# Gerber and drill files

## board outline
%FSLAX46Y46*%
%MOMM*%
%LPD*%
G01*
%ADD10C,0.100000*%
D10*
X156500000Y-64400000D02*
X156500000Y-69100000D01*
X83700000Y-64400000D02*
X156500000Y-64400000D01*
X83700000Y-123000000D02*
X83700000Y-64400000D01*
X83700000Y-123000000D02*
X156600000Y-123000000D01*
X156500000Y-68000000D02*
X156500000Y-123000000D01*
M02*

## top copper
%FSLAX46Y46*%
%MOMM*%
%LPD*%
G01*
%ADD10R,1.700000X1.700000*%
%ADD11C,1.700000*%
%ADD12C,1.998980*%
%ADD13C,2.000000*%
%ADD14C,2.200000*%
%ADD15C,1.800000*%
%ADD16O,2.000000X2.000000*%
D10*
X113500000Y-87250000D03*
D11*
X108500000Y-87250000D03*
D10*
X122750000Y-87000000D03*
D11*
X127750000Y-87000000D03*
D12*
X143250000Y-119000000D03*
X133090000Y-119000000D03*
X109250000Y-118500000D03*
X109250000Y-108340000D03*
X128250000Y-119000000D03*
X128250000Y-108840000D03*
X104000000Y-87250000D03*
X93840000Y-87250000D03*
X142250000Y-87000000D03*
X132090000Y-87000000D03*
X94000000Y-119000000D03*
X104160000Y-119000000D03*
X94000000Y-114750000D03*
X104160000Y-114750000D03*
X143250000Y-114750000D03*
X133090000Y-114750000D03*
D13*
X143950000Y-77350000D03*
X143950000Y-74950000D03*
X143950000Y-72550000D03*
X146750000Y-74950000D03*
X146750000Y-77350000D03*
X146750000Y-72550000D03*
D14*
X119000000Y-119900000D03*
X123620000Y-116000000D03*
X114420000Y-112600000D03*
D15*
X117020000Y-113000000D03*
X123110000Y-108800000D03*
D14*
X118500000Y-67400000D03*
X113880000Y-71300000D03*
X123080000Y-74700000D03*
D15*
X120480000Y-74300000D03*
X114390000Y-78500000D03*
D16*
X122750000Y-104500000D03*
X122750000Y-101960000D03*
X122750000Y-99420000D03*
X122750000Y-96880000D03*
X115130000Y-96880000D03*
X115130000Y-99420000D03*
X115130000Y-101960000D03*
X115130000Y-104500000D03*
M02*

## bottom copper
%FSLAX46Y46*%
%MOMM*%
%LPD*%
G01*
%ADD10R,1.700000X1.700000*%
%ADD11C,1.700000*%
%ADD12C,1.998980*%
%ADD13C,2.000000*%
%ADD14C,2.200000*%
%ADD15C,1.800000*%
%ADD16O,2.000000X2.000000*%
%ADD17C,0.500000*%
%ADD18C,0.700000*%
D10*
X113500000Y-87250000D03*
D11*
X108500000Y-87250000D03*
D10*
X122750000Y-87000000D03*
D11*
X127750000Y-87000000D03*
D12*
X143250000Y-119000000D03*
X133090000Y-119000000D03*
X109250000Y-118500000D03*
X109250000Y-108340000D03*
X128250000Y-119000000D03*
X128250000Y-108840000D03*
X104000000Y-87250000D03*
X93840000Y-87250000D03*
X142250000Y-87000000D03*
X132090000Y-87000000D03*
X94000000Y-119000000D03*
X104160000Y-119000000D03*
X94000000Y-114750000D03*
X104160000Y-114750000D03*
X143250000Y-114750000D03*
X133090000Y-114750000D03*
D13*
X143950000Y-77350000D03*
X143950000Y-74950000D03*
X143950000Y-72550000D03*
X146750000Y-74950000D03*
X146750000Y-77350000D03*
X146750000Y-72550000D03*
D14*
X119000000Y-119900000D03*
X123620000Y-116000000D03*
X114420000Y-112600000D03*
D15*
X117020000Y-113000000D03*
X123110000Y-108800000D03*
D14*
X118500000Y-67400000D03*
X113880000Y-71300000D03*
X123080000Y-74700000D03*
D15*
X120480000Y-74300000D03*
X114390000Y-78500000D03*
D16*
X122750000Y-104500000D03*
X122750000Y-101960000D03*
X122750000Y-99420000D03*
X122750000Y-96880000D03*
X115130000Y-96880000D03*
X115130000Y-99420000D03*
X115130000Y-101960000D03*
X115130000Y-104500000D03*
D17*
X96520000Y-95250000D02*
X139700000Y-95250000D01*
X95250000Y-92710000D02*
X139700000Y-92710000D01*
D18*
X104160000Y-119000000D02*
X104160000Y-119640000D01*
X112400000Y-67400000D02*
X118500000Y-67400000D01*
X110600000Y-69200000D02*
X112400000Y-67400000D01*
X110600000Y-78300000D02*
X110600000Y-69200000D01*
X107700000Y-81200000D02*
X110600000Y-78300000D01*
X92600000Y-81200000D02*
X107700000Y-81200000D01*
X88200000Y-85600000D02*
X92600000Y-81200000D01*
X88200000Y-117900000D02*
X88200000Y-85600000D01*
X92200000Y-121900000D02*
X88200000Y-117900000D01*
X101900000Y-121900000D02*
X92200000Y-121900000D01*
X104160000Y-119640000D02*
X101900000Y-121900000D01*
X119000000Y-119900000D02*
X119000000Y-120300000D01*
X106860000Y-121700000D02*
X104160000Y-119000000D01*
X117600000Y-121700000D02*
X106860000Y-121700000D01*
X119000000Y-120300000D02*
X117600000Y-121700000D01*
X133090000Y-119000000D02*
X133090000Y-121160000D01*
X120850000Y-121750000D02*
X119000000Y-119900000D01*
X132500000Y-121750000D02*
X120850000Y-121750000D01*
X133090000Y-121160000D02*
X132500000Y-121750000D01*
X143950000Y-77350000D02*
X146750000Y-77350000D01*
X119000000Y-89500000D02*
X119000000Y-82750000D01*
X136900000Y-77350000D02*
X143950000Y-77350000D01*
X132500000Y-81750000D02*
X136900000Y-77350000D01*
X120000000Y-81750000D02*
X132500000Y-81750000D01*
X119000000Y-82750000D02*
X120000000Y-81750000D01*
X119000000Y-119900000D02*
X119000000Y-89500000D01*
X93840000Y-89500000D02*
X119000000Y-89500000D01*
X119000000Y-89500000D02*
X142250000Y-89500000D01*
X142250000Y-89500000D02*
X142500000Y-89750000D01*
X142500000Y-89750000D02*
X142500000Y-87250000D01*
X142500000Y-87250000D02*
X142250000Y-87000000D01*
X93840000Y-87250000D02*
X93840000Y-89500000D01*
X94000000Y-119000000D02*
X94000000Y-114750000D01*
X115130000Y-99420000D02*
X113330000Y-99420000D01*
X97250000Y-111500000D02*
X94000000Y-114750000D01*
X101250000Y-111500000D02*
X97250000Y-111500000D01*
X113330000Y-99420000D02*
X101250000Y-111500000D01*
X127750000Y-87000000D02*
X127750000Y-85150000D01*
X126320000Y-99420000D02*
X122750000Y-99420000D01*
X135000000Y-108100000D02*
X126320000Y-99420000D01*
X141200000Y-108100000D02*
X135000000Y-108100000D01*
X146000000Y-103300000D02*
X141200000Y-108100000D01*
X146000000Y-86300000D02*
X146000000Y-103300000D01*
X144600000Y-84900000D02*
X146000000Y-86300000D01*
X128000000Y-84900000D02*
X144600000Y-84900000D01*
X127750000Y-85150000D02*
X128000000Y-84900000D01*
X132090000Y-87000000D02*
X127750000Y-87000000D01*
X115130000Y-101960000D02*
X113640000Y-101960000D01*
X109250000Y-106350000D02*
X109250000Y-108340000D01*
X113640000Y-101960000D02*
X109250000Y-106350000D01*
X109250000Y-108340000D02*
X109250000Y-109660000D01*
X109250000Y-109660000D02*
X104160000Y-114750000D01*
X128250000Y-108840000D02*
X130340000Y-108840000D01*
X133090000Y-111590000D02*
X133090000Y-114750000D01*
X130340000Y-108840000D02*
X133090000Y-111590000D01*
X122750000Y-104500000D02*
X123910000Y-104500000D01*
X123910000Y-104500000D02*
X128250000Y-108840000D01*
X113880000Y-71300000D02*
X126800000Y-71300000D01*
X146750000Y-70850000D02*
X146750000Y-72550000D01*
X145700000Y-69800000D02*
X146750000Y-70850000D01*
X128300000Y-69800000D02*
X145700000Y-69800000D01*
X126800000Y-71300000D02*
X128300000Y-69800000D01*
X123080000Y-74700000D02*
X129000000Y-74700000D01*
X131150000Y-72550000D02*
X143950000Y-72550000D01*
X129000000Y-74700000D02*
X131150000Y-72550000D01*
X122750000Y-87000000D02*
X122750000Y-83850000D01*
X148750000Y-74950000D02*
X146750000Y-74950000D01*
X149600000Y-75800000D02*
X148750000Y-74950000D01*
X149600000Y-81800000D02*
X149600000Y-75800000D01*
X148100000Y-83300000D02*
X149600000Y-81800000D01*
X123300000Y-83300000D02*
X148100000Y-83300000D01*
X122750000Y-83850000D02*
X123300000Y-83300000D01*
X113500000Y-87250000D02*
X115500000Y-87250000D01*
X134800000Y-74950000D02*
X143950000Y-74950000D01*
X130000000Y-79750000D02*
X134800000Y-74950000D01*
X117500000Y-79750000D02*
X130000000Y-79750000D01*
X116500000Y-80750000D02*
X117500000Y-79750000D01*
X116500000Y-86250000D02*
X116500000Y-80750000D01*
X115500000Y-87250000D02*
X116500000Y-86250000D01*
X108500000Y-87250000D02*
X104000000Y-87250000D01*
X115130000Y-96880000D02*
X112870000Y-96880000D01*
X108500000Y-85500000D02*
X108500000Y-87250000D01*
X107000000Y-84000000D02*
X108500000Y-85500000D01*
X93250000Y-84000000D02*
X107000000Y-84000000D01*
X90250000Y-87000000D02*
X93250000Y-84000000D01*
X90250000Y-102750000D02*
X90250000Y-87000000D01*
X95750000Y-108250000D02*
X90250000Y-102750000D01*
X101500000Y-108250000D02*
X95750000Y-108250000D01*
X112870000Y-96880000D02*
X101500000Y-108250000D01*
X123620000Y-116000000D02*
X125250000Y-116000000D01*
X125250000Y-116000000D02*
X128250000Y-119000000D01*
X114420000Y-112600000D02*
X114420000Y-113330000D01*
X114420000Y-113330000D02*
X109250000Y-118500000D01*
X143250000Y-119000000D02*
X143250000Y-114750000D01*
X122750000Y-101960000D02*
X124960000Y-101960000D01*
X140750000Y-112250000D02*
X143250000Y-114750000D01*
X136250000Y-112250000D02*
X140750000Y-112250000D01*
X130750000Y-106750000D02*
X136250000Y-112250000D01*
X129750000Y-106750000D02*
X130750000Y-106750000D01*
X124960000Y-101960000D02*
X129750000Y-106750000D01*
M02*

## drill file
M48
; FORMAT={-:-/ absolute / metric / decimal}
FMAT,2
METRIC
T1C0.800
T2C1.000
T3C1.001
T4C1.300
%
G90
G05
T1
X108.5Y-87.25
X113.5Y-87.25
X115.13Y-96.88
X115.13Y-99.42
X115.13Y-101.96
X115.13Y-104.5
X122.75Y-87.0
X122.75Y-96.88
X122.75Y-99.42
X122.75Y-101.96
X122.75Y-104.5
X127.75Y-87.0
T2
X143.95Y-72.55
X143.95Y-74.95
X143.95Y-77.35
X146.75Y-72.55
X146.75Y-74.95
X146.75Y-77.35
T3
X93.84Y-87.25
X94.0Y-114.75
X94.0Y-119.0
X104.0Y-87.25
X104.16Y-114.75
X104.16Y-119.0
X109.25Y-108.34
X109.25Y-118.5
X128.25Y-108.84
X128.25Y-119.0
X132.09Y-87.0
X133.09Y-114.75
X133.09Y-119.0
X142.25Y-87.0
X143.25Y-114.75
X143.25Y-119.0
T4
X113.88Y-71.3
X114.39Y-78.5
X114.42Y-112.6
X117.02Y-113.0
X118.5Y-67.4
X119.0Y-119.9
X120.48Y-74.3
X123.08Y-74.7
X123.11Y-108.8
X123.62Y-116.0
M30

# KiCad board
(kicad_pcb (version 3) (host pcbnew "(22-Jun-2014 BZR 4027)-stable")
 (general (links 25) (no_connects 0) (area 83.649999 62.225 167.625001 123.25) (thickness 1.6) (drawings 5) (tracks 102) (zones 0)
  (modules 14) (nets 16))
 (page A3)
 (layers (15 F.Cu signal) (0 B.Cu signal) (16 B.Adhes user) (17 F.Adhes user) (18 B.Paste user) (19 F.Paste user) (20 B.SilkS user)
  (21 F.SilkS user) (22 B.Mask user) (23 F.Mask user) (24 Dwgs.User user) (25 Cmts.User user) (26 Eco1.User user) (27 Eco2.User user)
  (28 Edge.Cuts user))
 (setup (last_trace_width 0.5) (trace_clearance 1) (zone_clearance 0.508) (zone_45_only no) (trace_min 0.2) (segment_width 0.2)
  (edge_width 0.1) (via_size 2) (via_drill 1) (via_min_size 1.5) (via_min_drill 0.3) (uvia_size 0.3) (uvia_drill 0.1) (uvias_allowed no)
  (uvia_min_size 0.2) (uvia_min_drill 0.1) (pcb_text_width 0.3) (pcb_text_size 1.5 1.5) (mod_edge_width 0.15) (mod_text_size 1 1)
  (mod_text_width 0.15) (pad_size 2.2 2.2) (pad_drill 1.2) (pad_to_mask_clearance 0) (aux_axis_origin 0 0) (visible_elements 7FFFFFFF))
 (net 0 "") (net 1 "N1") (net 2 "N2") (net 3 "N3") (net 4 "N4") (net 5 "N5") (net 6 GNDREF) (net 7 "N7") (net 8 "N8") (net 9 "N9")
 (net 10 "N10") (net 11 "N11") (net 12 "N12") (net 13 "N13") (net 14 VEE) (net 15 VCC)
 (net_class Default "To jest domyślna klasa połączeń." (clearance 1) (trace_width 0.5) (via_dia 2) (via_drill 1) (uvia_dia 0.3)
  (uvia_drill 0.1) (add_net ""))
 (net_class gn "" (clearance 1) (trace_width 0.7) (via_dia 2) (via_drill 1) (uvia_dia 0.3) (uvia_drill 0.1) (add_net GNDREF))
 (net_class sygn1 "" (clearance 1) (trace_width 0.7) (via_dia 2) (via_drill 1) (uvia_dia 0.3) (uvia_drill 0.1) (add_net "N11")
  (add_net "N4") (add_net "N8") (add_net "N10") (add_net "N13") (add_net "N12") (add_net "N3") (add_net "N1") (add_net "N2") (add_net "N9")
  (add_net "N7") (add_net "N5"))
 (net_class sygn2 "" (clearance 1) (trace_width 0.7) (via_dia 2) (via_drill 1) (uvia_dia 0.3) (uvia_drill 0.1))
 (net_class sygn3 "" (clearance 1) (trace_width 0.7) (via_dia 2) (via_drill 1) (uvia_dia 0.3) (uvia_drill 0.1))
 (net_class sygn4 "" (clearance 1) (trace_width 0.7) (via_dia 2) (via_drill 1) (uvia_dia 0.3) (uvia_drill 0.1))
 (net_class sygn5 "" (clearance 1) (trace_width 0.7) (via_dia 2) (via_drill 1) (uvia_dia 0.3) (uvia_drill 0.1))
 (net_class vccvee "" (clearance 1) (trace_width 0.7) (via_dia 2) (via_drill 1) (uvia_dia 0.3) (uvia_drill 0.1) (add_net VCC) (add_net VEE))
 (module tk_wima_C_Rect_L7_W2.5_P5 (layer F.Cu) (at 113.5 87.25 180)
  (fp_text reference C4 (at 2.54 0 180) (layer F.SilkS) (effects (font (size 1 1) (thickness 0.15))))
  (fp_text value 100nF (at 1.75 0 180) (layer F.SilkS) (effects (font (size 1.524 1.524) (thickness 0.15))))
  (pad 1 thru_hole rect (at 0 0 180) (size 1.7 1.7) (drill 0.8) (layers *.Cu *.Mask F.SilkS) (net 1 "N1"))
  (pad 2 thru_hole circle (at 5 0 180) (size 1.7 1.7) (drill 0.8) (layers *.Cu *.Mask F.SilkS) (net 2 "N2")))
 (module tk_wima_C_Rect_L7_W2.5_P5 (layer F.Cu) (at 122.75 87)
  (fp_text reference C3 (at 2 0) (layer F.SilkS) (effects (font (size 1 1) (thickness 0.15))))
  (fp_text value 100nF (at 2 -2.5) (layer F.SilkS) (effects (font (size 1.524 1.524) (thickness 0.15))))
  (pad 1 thru_hole rect (at 0 0) (size 1.7 1.7) (drill 0.8) (layers *.Cu *.Mask F.SilkS) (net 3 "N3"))
  (pad 2 thru_hole circle (at 5 0) (size 1.7 1.7) (drill 0.8) (layers *.Cu *.Mask F.SilkS) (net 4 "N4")))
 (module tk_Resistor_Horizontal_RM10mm (layer F.Cu) (at 143.25 119 180)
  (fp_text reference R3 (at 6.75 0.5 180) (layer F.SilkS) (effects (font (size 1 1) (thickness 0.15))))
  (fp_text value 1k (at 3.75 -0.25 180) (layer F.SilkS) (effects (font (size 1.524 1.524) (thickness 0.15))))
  (pad 1 thru_hole circle (at 0 0 180) (size 1.99898 1.99898) (drill 1.00076) (layers *.Cu *.SilkS *.Mask) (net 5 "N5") (clearance 1))
  (pad 2 thru_hole circle (at 10.16 0 180) (size 1.99898 1.99898) (drill 1.00076) (layers *.Cu *.SilkS *.Mask) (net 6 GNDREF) (clearance 1)))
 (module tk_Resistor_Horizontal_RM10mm (layer F.Cu) (at 109.25 118.5 90)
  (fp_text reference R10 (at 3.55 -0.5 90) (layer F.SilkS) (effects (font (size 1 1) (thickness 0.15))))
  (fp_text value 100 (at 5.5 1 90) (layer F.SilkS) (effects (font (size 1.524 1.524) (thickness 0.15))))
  (pad 1 thru_hole circle (at 0 0 90) (size 1.99898 1.99898) (drill 1.00076) (layers *.Cu *.SilkS *.Mask) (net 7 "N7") (clearance 1))
  (pad 2 thru_hole circle (at 10.16 0 90) (size 1.99898 1.99898) (drill 1.00076) (layers *.Cu *.SilkS *.Mask) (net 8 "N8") (clearance 1)))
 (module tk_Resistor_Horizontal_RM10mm (layer F.Cu) (at 128.25 119 90)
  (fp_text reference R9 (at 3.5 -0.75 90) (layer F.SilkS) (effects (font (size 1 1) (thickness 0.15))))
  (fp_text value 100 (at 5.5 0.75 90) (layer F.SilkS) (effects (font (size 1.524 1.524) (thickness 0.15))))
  (pad 1 thru_hole circle (at 0 0 90) (size 1.99898 1.99898) (drill 1.00076) (layers *.Cu *.SilkS *.Mask) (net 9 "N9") (clearance 1))
  (pad 2 thru_hole circle (at 10.16 0 90) (size 1.99898 1.99898) (drill 1.00076) (layers *.Cu *.SilkS *.Mask) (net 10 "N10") (clearance 1)))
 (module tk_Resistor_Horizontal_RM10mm (layer F.Cu) (at 104 87.25 180)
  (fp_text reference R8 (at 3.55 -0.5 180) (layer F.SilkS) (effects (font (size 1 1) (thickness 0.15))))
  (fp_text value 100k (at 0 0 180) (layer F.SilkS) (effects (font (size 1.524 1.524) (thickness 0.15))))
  (pad 1 thru_hole circle (at 0 0 180) (size 1.99898 1.99898) (drill 1.00076) (layers *.Cu *.SilkS *.Mask) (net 2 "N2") (clearance 1))
  (pad 2 thru_hole circle (at 10.16 0 180) (size 1.99898 1.99898) (drill 1.00076) (layers *.Cu *.SilkS *.Mask) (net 6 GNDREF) (clearance 1)))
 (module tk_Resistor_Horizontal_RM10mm (layer F.Cu) (at 142.25 87 180)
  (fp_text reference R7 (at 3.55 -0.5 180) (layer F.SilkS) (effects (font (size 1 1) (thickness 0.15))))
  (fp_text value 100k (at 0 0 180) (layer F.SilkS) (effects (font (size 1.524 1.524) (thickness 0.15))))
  (pad 1 thru_hole circle (at 0 0 180) (size 1.99898 1.99898) (drill 1.00076) (layers *.Cu *.SilkS *.Mask) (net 6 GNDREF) (clearance 1))
  (pad 2 thru_hole circle (at 10.16 0 180) (size 1.99898 1.99898) (drill 1.00076) (layers *.Cu *.SilkS *.Mask) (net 4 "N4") (clearance 1)))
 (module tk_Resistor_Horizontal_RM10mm (layer F.Cu) (at 94 119)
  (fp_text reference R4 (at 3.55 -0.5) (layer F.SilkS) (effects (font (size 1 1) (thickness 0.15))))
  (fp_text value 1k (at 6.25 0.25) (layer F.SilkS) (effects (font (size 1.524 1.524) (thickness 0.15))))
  (pad 1 thru_hole circle (at 0 0) (size 1.99898 1.99898) (drill 1.00076) (layers *.Cu *.SilkS *.Mask) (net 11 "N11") (clearance 1))
  (pad 2 thru_hole circle (at 10.16 0) (size 1.99898 1.99898) (drill 1.00076) (layers *.Cu *.SilkS *.Mask) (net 6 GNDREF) (clearance 1)))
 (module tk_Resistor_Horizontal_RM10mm (layer F.Cu) (at 94 114.75)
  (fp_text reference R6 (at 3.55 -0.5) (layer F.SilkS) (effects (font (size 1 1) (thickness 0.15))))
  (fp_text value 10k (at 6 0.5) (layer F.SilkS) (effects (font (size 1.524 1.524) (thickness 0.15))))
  (pad 1 thru_hole circle (at 0 0) (size 1.99898 1.99898) (drill 1.00076) (layers *.Cu *.SilkS *.Mask) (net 11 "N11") (clearance 1))
  (pad 2 thru_hole circle (at 10.16 0) (size 1.99898 1.99898) (drill 1.00076) (layers *.Cu *.SilkS *.Mask) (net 8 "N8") (clearance 1)))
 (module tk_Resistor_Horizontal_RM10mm (layer F.Cu) (at 143.25 114.75 180)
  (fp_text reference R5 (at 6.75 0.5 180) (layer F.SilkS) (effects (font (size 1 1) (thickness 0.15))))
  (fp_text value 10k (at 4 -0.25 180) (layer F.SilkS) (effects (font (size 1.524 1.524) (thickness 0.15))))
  (pad 1 thru_hole circle (at 0 0 180) (size 1.99898 1.99898) (drill 1.00076) (layers *.Cu *.SilkS *.Mask) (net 5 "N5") (clearance 1))
  (pad 2 thru_hole circle (at 10.16 0 180) (size 1.99898 1.99898) (drill 1.00076) (layers *.Cu *.SilkS *.Mask) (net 10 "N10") (clearance 1)))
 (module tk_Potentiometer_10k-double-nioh (layer F.Cu) (at 151.25 73 90)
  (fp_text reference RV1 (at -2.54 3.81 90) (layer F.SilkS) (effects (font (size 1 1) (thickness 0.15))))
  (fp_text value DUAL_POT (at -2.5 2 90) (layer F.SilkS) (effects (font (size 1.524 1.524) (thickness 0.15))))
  (pad 4 thru_hole circle (at -4.35 -7.3) (size 2 2) (drill 1) (layers *.Cu *.Mask F.SilkS) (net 6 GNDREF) (clearance 1))
  (pad 5 thru_hole circle (at -1.95 -7.3) (size 2 2) (drill 1) (layers *.Cu *.Mask F.SilkS) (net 1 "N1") (clearance 1))
  (pad 6 thru_hole circle (at 0.45 -7.3) (size 2 2) (drill 1) (layers *.Cu *.Mask F.SilkS) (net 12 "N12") (clearance 1))
  (pad 2 thru_hole circle (at -1.95 -4.5) (size 2 2) (drill 1) (layers *.Cu *.Mask F.SilkS) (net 3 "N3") (clearance 1))
  (pad 1 thru_hole circle (at -4.35 -4.5) (size 2 2) (drill 1) (layers *.Cu *.Mask F.SilkS) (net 6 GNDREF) (clearance 1))
  (pad 3 thru_hole circle (at 0.45 -4.5) (size 2 2) (drill 1) (layers *.Cu *.Mask F.SilkS) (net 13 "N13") (clearance 1)))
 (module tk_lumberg (layer F.Cu) (at 119 122)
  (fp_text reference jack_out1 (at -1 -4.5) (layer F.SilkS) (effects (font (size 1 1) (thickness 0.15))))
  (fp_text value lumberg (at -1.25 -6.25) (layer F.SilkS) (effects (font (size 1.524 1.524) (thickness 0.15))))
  (pad 1 thru_hole circle (at 0 -2.1) (size 2.2 2.2) (drill 1.3) (layers *.Cu *.Mask F.SilkS) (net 6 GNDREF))
  (pad 2 thru_hole circle (at 4.62 -6) (size 2.2 2.2) (drill 1.3) (layers *.Cu *.Mask F.SilkS) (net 9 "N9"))
  (pad 3 thru_hole circle (at -4.58 -9.4) (size 2.2 2.2) (drill 1.3) (layers *.Cu *.Mask F.SilkS) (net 7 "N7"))
  (pad 4 thru_hole circle (at -1.98 -9) (size 1.8 1.8) (drill 1.3) (layers *.Cu *.Mask F.SilkS))
  (pad 5 thru_hole circle (at 4.11 -13.2) (size 1.8 1.8) (drill 1.3) (layers *.Cu *.Mask F.SilkS)))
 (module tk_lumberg (layer F.Cu) (at 118.5 65.3 180)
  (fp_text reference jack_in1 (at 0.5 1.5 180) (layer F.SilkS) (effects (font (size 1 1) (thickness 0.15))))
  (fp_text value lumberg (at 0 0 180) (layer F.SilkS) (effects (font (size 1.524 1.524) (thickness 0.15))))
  (pad 1 thru_hole circle (at 0 -2.1 180) (size 2.2 2.2) (drill 1.3) (layers *.Cu *.Mask F.SilkS) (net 6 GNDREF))
  (pad 2 thru_hole circle (at 4.62 -6 180) (size 2.2 2.2) (drill 1.3) (layers *.Cu *.Mask F.SilkS) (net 13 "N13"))
  (pad 3 thru_hole circle (at -4.58 -9.4 180) (size 2.2 2.2) (drill 1.3) (layers *.Cu *.Mask F.SilkS) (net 12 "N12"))
  (pad 4 thru_hole circle (at -1.98 -9 180) (size 1.8 1.8) (drill 1.3) (layers *.Cu *.Mask F.SilkS))
  (pad 5 thru_hole circle (at 4.11 -13.2 180) (size 1.8 1.8) (drill 1.3) (layers *.Cu *.Mask F.SilkS)))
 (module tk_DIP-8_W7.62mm (layer F.Cu) (at 122.75 104.5 180) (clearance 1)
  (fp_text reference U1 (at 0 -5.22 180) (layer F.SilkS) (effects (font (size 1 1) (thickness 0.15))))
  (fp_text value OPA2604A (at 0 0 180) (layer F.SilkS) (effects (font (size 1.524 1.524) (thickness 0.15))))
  (pad 1 thru_hole oval (at 0 0 180) (size 2 2) (drill 0.8) (layers *.Cu *.Mask F.SilkS) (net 10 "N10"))
  (pad 2 thru_hole oval (at 0 2.54 180) (size 2 2) (drill 0.8) (layers *.Cu *.Mask F.SilkS) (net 5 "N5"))
  (pad 3 thru_hole oval (at 0 5.08 180) (size 2 2) (drill 0.8) (layers *.Cu *.Mask F.SilkS) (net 4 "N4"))
  (pad 4 thru_hole oval (at 0 7.62 180) (size 2 2) (drill 0.8) (layers *.Cu *.Mask F.SilkS) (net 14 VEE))
  (pad 5 thru_hole oval (at 7.62 7.62 180) (size 2 2) (drill 0.8) (layers *.Cu *.Mask F.SilkS) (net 2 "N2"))
  (pad 6 thru_hole oval (at 7.62 5.08 180) (size 2 2) (drill 0.8) (layers *.Cu *.Mask F.SilkS) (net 11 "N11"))
  (pad 7 thru_hole oval (at 7.62 2.54 180) (size 2 2) (drill 0.8) (layers *.Cu *.Mask F.SilkS) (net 8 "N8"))
  (pad 8 thru_hole oval (at 7.62 0 180) (size 2 2) (drill 0.8) (layers *.Cu *.Mask F.SilkS) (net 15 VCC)))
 (gr_line (start 156.5 64.4) (end 156.5 69.1) (angle 90) (layer Edge.Cuts) (width 0.1))
 (gr_line (start 83.7 64.4) (end 156.5 64.4) (angle 90) (layer Edge.Cuts) (width 0.1))
 (gr_line (start 83.7 123) (end 83.7 64.4) (angle 90) (layer Edge.Cuts) (width 0.1))
 (gr_line (start 83.7 123) (end 156.6 123) (angle 90) (layer Edge.Cuts) (width 0.1))
 (gr_line (start 156.5 68) (end 156.5 123) (angle 90) (layer Edge.Cuts) (width 0.1))
 (segment (start 96.52 95.25) (end 139.7 95.25) (width 0.5) (layer B.Cu) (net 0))
 (segment (start 95.25 92.71) (end 139.7 92.71) (width 0.5) (layer B.Cu) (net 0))
 (segment (start 104.16 119) (end 104.16 119.64) (width 0.7) (layer B.Cu) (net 6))
 (segment (start 112.4 67.4) (end 118.5 67.4) (width 0.7) (layer B.Cu) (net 6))
 (segment (start 110.6 69.2) (end 112.4 67.4) (width 0.7) (layer B.Cu) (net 6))
 (segment (start 110.6 78.3) (end 110.6 69.2) (width 0.7) (layer B.Cu) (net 6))
 (segment (start 107.7 81.2) (end 110.6 78.3) (width 0.7) (layer B.Cu) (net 6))
 (segment (start 92.6 81.2) (end 107.7 81.2) (width 0.7) (layer B.Cu) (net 6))
 (segment (start 88.2 85.6) (end 92.6 81.2) (width 0.7) (layer B.Cu) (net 6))
 (segment (start 88.2 117.9) (end 88.2 85.6) (width 0.7) (layer B.Cu) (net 6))
 (segment (start 92.2 121.9) (end 88.2 117.9) (width 0.7) (layer B.Cu) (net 6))
 (segment (start 101.9 121.9) (end 92.2 121.9) (width 0.7) (layer B.Cu) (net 6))
 (segment (start 104.16 119.64) (end 101.9 121.9) (width 0.7) (layer B.Cu) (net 6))
 (segment (start 119 119.9) (end 119 120.3) (width 0.7) (layer B.Cu) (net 6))
 (segment (start 106.86 121.7) (end 104.16 119) (width 0.7) (layer B.Cu) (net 6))
 (segment (start 117.6 121.7) (end 106.86 121.7) (width 0.7) (layer B.Cu) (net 6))
 (segment (start 119 120.3) (end 117.6 121.7) (width 0.7) (layer B.Cu) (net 6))
 (segment (start 133.09 119) (end 133.09 121.16) (width 0.7) (layer B.Cu) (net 6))
 (segment (start 120.85 121.75) (end 119 119.9) (width 0.7) (layer B.Cu) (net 6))
 (segment (start 132.5 121.75) (end 120.85 121.75) (width 0.7) (layer B.Cu) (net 6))
 (segment (start 133.09 121.16) (end 132.5 121.75) (width 0.7) (layer B.Cu) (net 6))
 (segment (start 143.95 77.35) (end 146.75 77.35) (width 0.7) (layer B.Cu) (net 6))
 (segment (start 119 89.5) (end 119 82.75) (width 0.7) (layer B.Cu) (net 6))
 (segment (start 136.9 77.35) (end 143.95 77.35) (width 0.7) (layer B.Cu) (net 6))
 (segment (start 132.5 81.75) (end 136.9 77.35) (width 0.7) (layer B.Cu) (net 6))
 (segment (start 120 81.75) (end 132.5 81.75) (width 0.7) (layer B.Cu) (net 6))
 (segment (start 119 82.75) (end 120 81.75) (width 0.7) (layer B.Cu) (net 6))
 (segment (start 119 119.9) (end 119 89.5) (width 0.7) (layer B.Cu) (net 6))
 (segment (start 93.84 89.5) (end 119 89.5) (width 0.7) (layer B.Cu) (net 6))
 (segment (start 119 89.5) (end 142.25 89.5) (width 0.7) (layer B.Cu) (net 6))
 (segment (start 142.25 89.5) (end 142.5 89.75) (width 0.7) (layer B.Cu) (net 6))
 (segment (start 142.5 89.75) (end 142.5 87.25) (width 0.7) (layer B.Cu) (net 6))
 (segment (start 142.5 87.25) (end 142.25 87) (width 0.7) (layer B.Cu) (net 6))
 (segment (start 93.84 87.25) (end 93.84 89.5) (width 0.7) (layer B.Cu) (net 6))
 (segment (start 94 119) (end 94 114.75) (width 0.7) (layer B.Cu) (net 11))
 (segment (start 115.13 99.42) (end 113.33 99.42) (width 0.7) (layer B.Cu) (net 11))
 (segment (start 97.25 111.5) (end 94 114.75) (width 0.7) (layer B.Cu) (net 11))
 (segment (start 101.25 111.5) (end 97.25 111.5) (width 0.7) (layer B.Cu) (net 11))
 (segment (start 113.33 99.42) (end 101.25 111.5) (width 0.7) (layer B.Cu) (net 11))
 (segment (start 127.75 87) (end 127.75 85.15) (width 0.7) (layer B.Cu) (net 4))
 (segment (start 126.32 99.42) (end 122.75 99.42) (width 0.7) (layer B.Cu) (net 4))
 (segment (start 135 108.1) (end 126.32 99.42) (width 0.7) (layer B.Cu) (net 4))
 (segment (start 141.2 108.1) (end 135 108.1) (width 0.7) (layer B.Cu) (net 4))
 (segment (start 146 103.3) (end 141.2 108.1) (width 0.7) (layer B.Cu) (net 4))
 (segment (start 146 86.3) (end 146 103.3) (width 0.7) (layer B.Cu) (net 4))
 (segment (start 144.6 84.9) (end 146 86.3) (width 0.7) (layer B.Cu) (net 4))
 (segment (start 128 84.9) (end 144.6 84.9) (width 0.7) (layer B.Cu) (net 4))
 (segment (start 127.75 85.15) (end 128 84.9) (width 0.7) (layer B.Cu) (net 4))
 (segment (start 132.09 87) (end 127.75 87) (width 0.7) (layer B.Cu) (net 4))
 (segment (start 115.13 101.96) (end 113.64 101.96) (width 0.7) (layer B.Cu) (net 8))
 (segment (start 109.25 106.35) (end 109.25 108.34) (width 0.7) (layer B.Cu) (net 8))
 (segment (start 113.64 101.96) (end 109.25 106.35) (width 0.7) (layer B.Cu) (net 8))
 (segment (start 109.25 108.34) (end 109.25 109.66) (width 0.7) (layer B.Cu) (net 8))
 (segment (start 109.25 109.66) (end 104.16 114.75) (width 0.7) (layer B.Cu) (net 8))
 (segment (start 128.25 108.84) (end 130.34 108.84) (width 0.7) (layer B.Cu) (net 10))
 (segment (start 133.09 111.59) (end 133.09 114.75) (width 0.7) (layer B.Cu) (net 10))
 (segment (start 130.34 108.84) (end 133.09 111.59) (width 0.7) (layer B.Cu) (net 10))
 (segment (start 122.75 104.5) (end 123.91 104.5) (width 0.7) (layer B.Cu) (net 10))
 (segment (start 123.91 104.5) (end 128.25 108.84) (width 0.7) (layer B.Cu) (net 10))
 (segment (start 113.88 71.3) (end 126.8 71.3) (width 0.7) (layer B.Cu) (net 13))
 (segment (start 146.75 70.85) (end 146.75 72.55) (width 0.7) (layer B.Cu) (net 13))
 (segment (start 145.7 69.8) (end 146.75 70.85) (width 0.7) (layer B.Cu) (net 13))
 (segment (start 128.3 69.8) (end 145.7 69.8) (width 0.7) (layer B.Cu) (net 13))
 (segment (start 126.8 71.3) (end 128.3 69.8) (width 0.7) (layer B.Cu) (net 13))
 (segment (start 123.08 74.7) (end 129 74.7) (width 0.7) (layer B.Cu) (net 12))
 (segment (start 131.15 72.55) (end 143.95 72.55) (width 0.7) (layer B.Cu) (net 12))
 (segment (start 129 74.7) (end 131.15 72.55) (width 0.7) (layer B.Cu) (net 12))
 (segment (start 122.75 87) (end 122.75 83.85) (width 0.7) (layer B.Cu) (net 3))
 (segment (start 148.75 74.95) (end 146.75 74.95) (width 0.7) (layer B.Cu) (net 3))
 (segment (start 149.6 75.8) (end 148.75 74.95) (width 0.7) (layer B.Cu) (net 3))
 (segment (start 149.6 81.8) (end 149.6 75.8) (width 0.7) (layer B.Cu) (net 3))
 (segment (start 148.1 83.3) (end 149.6 81.8) (width 0.7) (layer B.Cu) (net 3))
 (segment (start 123.3 83.3) (end 148.1 83.3) (width 0.7) (layer B.Cu) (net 3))
 (segment (start 122.75 83.85) (end 123.3 83.3) (width 0.7) (layer B.Cu) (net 3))
 (segment (start 113.5 87.25) (end 115.5 87.25) (width 0.7) (layer B.Cu) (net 1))
 (segment (start 134.8 74.95) (end 143.95 74.95) (width 0.7) (layer B.Cu) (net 1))
 (segment (start 130 79.75) (end 134.8 74.95) (width 0.7) (layer B.Cu) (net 1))
 (segment (start 117.5 79.75) (end 130 79.75) (width 0.7) (layer B.Cu) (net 1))
 (segment (start 116.5 80.75) (end 117.5 79.75) (width 0.7) (layer B.Cu) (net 1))
 (segment (start 116.5 86.25) (end 116.5 80.75) (width 0.7) (layer B.Cu) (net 1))
 (segment (start 115.5 87.25) (end 116.5 86.25) (width 0.7) (layer B.Cu) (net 1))
 (segment (start 108.5 87.25) (end 104 87.25) (width 0.7) (layer B.Cu) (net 2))
 (segment (start 115.13 96.88) (end 112.87 96.88) (width 0.7) (layer B.Cu) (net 2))
 (segment (start 108.5 85.5) (end 108.5 87.25) (width 0.7) (layer B.Cu) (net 2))
 (segment (start 107 84) (end 108.5 85.5) (width 0.7) (layer B.Cu) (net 2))
 (segment (start 93.25 84) (end 107 84) (width 0.7) (layer B.Cu) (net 2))
 (segment (start 90.25 87) (end 93.25 84) (width 0.7) (layer B.Cu) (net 2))
 (segment (start 90.25 102.75) (end 90.25 87) (width 0.7) (layer B.Cu) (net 2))
 (segment (start 95.75 108.25) (end 90.25 102.75) (width 0.7) (layer B.Cu) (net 2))
 (segment (start 101.5 108.25) (end 95.75 108.25) (width 0.7) (layer B.Cu) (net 2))
 (segment (start 112.87 96.88) (end 101.5 108.25) (width 0.7) (layer B.Cu) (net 2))
 (segment (start 123.62 116) (end 125.25 116) (width 0.7) (layer B.Cu) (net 9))
 (segment (start 125.25 116) (end 128.25 119) (width 0.7) (layer B.Cu) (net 9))
 (segment (start 114.42 112.6) (end 114.42 113.33) (width 0.7) (layer B.Cu) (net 7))
 (segment (start 114.42 113.33) (end 109.25 118.5) (width 0.7) (layer B.Cu) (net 7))
 (segment (start 143.25 119) (end 143.25 114.75) (width 0.7) (layer B.Cu) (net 5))
 (segment (start 122.75 101.96) (end 124.96 101.96) (width 0.7) (layer B.Cu) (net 5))
 (segment (start 140.75 112.25) (end 143.25 114.75) (width 0.7) (layer B.Cu) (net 5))
 (segment (start 136.25 112.25) (end 140.75 112.25) (width 0.7) (layer B.Cu) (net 5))
 (segment (start 130.75 106.75) (end 136.25 112.25) (width 0.7) (layer B.Cu) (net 5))
 (segment (start 129.75 106.75) (end 130.75 106.75) (width 0.7) (layer B.Cu) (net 5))
 (segment (start 124.96 101.96) (end 129.75 106.75) (width 0.7) (layer B.Cu) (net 5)))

